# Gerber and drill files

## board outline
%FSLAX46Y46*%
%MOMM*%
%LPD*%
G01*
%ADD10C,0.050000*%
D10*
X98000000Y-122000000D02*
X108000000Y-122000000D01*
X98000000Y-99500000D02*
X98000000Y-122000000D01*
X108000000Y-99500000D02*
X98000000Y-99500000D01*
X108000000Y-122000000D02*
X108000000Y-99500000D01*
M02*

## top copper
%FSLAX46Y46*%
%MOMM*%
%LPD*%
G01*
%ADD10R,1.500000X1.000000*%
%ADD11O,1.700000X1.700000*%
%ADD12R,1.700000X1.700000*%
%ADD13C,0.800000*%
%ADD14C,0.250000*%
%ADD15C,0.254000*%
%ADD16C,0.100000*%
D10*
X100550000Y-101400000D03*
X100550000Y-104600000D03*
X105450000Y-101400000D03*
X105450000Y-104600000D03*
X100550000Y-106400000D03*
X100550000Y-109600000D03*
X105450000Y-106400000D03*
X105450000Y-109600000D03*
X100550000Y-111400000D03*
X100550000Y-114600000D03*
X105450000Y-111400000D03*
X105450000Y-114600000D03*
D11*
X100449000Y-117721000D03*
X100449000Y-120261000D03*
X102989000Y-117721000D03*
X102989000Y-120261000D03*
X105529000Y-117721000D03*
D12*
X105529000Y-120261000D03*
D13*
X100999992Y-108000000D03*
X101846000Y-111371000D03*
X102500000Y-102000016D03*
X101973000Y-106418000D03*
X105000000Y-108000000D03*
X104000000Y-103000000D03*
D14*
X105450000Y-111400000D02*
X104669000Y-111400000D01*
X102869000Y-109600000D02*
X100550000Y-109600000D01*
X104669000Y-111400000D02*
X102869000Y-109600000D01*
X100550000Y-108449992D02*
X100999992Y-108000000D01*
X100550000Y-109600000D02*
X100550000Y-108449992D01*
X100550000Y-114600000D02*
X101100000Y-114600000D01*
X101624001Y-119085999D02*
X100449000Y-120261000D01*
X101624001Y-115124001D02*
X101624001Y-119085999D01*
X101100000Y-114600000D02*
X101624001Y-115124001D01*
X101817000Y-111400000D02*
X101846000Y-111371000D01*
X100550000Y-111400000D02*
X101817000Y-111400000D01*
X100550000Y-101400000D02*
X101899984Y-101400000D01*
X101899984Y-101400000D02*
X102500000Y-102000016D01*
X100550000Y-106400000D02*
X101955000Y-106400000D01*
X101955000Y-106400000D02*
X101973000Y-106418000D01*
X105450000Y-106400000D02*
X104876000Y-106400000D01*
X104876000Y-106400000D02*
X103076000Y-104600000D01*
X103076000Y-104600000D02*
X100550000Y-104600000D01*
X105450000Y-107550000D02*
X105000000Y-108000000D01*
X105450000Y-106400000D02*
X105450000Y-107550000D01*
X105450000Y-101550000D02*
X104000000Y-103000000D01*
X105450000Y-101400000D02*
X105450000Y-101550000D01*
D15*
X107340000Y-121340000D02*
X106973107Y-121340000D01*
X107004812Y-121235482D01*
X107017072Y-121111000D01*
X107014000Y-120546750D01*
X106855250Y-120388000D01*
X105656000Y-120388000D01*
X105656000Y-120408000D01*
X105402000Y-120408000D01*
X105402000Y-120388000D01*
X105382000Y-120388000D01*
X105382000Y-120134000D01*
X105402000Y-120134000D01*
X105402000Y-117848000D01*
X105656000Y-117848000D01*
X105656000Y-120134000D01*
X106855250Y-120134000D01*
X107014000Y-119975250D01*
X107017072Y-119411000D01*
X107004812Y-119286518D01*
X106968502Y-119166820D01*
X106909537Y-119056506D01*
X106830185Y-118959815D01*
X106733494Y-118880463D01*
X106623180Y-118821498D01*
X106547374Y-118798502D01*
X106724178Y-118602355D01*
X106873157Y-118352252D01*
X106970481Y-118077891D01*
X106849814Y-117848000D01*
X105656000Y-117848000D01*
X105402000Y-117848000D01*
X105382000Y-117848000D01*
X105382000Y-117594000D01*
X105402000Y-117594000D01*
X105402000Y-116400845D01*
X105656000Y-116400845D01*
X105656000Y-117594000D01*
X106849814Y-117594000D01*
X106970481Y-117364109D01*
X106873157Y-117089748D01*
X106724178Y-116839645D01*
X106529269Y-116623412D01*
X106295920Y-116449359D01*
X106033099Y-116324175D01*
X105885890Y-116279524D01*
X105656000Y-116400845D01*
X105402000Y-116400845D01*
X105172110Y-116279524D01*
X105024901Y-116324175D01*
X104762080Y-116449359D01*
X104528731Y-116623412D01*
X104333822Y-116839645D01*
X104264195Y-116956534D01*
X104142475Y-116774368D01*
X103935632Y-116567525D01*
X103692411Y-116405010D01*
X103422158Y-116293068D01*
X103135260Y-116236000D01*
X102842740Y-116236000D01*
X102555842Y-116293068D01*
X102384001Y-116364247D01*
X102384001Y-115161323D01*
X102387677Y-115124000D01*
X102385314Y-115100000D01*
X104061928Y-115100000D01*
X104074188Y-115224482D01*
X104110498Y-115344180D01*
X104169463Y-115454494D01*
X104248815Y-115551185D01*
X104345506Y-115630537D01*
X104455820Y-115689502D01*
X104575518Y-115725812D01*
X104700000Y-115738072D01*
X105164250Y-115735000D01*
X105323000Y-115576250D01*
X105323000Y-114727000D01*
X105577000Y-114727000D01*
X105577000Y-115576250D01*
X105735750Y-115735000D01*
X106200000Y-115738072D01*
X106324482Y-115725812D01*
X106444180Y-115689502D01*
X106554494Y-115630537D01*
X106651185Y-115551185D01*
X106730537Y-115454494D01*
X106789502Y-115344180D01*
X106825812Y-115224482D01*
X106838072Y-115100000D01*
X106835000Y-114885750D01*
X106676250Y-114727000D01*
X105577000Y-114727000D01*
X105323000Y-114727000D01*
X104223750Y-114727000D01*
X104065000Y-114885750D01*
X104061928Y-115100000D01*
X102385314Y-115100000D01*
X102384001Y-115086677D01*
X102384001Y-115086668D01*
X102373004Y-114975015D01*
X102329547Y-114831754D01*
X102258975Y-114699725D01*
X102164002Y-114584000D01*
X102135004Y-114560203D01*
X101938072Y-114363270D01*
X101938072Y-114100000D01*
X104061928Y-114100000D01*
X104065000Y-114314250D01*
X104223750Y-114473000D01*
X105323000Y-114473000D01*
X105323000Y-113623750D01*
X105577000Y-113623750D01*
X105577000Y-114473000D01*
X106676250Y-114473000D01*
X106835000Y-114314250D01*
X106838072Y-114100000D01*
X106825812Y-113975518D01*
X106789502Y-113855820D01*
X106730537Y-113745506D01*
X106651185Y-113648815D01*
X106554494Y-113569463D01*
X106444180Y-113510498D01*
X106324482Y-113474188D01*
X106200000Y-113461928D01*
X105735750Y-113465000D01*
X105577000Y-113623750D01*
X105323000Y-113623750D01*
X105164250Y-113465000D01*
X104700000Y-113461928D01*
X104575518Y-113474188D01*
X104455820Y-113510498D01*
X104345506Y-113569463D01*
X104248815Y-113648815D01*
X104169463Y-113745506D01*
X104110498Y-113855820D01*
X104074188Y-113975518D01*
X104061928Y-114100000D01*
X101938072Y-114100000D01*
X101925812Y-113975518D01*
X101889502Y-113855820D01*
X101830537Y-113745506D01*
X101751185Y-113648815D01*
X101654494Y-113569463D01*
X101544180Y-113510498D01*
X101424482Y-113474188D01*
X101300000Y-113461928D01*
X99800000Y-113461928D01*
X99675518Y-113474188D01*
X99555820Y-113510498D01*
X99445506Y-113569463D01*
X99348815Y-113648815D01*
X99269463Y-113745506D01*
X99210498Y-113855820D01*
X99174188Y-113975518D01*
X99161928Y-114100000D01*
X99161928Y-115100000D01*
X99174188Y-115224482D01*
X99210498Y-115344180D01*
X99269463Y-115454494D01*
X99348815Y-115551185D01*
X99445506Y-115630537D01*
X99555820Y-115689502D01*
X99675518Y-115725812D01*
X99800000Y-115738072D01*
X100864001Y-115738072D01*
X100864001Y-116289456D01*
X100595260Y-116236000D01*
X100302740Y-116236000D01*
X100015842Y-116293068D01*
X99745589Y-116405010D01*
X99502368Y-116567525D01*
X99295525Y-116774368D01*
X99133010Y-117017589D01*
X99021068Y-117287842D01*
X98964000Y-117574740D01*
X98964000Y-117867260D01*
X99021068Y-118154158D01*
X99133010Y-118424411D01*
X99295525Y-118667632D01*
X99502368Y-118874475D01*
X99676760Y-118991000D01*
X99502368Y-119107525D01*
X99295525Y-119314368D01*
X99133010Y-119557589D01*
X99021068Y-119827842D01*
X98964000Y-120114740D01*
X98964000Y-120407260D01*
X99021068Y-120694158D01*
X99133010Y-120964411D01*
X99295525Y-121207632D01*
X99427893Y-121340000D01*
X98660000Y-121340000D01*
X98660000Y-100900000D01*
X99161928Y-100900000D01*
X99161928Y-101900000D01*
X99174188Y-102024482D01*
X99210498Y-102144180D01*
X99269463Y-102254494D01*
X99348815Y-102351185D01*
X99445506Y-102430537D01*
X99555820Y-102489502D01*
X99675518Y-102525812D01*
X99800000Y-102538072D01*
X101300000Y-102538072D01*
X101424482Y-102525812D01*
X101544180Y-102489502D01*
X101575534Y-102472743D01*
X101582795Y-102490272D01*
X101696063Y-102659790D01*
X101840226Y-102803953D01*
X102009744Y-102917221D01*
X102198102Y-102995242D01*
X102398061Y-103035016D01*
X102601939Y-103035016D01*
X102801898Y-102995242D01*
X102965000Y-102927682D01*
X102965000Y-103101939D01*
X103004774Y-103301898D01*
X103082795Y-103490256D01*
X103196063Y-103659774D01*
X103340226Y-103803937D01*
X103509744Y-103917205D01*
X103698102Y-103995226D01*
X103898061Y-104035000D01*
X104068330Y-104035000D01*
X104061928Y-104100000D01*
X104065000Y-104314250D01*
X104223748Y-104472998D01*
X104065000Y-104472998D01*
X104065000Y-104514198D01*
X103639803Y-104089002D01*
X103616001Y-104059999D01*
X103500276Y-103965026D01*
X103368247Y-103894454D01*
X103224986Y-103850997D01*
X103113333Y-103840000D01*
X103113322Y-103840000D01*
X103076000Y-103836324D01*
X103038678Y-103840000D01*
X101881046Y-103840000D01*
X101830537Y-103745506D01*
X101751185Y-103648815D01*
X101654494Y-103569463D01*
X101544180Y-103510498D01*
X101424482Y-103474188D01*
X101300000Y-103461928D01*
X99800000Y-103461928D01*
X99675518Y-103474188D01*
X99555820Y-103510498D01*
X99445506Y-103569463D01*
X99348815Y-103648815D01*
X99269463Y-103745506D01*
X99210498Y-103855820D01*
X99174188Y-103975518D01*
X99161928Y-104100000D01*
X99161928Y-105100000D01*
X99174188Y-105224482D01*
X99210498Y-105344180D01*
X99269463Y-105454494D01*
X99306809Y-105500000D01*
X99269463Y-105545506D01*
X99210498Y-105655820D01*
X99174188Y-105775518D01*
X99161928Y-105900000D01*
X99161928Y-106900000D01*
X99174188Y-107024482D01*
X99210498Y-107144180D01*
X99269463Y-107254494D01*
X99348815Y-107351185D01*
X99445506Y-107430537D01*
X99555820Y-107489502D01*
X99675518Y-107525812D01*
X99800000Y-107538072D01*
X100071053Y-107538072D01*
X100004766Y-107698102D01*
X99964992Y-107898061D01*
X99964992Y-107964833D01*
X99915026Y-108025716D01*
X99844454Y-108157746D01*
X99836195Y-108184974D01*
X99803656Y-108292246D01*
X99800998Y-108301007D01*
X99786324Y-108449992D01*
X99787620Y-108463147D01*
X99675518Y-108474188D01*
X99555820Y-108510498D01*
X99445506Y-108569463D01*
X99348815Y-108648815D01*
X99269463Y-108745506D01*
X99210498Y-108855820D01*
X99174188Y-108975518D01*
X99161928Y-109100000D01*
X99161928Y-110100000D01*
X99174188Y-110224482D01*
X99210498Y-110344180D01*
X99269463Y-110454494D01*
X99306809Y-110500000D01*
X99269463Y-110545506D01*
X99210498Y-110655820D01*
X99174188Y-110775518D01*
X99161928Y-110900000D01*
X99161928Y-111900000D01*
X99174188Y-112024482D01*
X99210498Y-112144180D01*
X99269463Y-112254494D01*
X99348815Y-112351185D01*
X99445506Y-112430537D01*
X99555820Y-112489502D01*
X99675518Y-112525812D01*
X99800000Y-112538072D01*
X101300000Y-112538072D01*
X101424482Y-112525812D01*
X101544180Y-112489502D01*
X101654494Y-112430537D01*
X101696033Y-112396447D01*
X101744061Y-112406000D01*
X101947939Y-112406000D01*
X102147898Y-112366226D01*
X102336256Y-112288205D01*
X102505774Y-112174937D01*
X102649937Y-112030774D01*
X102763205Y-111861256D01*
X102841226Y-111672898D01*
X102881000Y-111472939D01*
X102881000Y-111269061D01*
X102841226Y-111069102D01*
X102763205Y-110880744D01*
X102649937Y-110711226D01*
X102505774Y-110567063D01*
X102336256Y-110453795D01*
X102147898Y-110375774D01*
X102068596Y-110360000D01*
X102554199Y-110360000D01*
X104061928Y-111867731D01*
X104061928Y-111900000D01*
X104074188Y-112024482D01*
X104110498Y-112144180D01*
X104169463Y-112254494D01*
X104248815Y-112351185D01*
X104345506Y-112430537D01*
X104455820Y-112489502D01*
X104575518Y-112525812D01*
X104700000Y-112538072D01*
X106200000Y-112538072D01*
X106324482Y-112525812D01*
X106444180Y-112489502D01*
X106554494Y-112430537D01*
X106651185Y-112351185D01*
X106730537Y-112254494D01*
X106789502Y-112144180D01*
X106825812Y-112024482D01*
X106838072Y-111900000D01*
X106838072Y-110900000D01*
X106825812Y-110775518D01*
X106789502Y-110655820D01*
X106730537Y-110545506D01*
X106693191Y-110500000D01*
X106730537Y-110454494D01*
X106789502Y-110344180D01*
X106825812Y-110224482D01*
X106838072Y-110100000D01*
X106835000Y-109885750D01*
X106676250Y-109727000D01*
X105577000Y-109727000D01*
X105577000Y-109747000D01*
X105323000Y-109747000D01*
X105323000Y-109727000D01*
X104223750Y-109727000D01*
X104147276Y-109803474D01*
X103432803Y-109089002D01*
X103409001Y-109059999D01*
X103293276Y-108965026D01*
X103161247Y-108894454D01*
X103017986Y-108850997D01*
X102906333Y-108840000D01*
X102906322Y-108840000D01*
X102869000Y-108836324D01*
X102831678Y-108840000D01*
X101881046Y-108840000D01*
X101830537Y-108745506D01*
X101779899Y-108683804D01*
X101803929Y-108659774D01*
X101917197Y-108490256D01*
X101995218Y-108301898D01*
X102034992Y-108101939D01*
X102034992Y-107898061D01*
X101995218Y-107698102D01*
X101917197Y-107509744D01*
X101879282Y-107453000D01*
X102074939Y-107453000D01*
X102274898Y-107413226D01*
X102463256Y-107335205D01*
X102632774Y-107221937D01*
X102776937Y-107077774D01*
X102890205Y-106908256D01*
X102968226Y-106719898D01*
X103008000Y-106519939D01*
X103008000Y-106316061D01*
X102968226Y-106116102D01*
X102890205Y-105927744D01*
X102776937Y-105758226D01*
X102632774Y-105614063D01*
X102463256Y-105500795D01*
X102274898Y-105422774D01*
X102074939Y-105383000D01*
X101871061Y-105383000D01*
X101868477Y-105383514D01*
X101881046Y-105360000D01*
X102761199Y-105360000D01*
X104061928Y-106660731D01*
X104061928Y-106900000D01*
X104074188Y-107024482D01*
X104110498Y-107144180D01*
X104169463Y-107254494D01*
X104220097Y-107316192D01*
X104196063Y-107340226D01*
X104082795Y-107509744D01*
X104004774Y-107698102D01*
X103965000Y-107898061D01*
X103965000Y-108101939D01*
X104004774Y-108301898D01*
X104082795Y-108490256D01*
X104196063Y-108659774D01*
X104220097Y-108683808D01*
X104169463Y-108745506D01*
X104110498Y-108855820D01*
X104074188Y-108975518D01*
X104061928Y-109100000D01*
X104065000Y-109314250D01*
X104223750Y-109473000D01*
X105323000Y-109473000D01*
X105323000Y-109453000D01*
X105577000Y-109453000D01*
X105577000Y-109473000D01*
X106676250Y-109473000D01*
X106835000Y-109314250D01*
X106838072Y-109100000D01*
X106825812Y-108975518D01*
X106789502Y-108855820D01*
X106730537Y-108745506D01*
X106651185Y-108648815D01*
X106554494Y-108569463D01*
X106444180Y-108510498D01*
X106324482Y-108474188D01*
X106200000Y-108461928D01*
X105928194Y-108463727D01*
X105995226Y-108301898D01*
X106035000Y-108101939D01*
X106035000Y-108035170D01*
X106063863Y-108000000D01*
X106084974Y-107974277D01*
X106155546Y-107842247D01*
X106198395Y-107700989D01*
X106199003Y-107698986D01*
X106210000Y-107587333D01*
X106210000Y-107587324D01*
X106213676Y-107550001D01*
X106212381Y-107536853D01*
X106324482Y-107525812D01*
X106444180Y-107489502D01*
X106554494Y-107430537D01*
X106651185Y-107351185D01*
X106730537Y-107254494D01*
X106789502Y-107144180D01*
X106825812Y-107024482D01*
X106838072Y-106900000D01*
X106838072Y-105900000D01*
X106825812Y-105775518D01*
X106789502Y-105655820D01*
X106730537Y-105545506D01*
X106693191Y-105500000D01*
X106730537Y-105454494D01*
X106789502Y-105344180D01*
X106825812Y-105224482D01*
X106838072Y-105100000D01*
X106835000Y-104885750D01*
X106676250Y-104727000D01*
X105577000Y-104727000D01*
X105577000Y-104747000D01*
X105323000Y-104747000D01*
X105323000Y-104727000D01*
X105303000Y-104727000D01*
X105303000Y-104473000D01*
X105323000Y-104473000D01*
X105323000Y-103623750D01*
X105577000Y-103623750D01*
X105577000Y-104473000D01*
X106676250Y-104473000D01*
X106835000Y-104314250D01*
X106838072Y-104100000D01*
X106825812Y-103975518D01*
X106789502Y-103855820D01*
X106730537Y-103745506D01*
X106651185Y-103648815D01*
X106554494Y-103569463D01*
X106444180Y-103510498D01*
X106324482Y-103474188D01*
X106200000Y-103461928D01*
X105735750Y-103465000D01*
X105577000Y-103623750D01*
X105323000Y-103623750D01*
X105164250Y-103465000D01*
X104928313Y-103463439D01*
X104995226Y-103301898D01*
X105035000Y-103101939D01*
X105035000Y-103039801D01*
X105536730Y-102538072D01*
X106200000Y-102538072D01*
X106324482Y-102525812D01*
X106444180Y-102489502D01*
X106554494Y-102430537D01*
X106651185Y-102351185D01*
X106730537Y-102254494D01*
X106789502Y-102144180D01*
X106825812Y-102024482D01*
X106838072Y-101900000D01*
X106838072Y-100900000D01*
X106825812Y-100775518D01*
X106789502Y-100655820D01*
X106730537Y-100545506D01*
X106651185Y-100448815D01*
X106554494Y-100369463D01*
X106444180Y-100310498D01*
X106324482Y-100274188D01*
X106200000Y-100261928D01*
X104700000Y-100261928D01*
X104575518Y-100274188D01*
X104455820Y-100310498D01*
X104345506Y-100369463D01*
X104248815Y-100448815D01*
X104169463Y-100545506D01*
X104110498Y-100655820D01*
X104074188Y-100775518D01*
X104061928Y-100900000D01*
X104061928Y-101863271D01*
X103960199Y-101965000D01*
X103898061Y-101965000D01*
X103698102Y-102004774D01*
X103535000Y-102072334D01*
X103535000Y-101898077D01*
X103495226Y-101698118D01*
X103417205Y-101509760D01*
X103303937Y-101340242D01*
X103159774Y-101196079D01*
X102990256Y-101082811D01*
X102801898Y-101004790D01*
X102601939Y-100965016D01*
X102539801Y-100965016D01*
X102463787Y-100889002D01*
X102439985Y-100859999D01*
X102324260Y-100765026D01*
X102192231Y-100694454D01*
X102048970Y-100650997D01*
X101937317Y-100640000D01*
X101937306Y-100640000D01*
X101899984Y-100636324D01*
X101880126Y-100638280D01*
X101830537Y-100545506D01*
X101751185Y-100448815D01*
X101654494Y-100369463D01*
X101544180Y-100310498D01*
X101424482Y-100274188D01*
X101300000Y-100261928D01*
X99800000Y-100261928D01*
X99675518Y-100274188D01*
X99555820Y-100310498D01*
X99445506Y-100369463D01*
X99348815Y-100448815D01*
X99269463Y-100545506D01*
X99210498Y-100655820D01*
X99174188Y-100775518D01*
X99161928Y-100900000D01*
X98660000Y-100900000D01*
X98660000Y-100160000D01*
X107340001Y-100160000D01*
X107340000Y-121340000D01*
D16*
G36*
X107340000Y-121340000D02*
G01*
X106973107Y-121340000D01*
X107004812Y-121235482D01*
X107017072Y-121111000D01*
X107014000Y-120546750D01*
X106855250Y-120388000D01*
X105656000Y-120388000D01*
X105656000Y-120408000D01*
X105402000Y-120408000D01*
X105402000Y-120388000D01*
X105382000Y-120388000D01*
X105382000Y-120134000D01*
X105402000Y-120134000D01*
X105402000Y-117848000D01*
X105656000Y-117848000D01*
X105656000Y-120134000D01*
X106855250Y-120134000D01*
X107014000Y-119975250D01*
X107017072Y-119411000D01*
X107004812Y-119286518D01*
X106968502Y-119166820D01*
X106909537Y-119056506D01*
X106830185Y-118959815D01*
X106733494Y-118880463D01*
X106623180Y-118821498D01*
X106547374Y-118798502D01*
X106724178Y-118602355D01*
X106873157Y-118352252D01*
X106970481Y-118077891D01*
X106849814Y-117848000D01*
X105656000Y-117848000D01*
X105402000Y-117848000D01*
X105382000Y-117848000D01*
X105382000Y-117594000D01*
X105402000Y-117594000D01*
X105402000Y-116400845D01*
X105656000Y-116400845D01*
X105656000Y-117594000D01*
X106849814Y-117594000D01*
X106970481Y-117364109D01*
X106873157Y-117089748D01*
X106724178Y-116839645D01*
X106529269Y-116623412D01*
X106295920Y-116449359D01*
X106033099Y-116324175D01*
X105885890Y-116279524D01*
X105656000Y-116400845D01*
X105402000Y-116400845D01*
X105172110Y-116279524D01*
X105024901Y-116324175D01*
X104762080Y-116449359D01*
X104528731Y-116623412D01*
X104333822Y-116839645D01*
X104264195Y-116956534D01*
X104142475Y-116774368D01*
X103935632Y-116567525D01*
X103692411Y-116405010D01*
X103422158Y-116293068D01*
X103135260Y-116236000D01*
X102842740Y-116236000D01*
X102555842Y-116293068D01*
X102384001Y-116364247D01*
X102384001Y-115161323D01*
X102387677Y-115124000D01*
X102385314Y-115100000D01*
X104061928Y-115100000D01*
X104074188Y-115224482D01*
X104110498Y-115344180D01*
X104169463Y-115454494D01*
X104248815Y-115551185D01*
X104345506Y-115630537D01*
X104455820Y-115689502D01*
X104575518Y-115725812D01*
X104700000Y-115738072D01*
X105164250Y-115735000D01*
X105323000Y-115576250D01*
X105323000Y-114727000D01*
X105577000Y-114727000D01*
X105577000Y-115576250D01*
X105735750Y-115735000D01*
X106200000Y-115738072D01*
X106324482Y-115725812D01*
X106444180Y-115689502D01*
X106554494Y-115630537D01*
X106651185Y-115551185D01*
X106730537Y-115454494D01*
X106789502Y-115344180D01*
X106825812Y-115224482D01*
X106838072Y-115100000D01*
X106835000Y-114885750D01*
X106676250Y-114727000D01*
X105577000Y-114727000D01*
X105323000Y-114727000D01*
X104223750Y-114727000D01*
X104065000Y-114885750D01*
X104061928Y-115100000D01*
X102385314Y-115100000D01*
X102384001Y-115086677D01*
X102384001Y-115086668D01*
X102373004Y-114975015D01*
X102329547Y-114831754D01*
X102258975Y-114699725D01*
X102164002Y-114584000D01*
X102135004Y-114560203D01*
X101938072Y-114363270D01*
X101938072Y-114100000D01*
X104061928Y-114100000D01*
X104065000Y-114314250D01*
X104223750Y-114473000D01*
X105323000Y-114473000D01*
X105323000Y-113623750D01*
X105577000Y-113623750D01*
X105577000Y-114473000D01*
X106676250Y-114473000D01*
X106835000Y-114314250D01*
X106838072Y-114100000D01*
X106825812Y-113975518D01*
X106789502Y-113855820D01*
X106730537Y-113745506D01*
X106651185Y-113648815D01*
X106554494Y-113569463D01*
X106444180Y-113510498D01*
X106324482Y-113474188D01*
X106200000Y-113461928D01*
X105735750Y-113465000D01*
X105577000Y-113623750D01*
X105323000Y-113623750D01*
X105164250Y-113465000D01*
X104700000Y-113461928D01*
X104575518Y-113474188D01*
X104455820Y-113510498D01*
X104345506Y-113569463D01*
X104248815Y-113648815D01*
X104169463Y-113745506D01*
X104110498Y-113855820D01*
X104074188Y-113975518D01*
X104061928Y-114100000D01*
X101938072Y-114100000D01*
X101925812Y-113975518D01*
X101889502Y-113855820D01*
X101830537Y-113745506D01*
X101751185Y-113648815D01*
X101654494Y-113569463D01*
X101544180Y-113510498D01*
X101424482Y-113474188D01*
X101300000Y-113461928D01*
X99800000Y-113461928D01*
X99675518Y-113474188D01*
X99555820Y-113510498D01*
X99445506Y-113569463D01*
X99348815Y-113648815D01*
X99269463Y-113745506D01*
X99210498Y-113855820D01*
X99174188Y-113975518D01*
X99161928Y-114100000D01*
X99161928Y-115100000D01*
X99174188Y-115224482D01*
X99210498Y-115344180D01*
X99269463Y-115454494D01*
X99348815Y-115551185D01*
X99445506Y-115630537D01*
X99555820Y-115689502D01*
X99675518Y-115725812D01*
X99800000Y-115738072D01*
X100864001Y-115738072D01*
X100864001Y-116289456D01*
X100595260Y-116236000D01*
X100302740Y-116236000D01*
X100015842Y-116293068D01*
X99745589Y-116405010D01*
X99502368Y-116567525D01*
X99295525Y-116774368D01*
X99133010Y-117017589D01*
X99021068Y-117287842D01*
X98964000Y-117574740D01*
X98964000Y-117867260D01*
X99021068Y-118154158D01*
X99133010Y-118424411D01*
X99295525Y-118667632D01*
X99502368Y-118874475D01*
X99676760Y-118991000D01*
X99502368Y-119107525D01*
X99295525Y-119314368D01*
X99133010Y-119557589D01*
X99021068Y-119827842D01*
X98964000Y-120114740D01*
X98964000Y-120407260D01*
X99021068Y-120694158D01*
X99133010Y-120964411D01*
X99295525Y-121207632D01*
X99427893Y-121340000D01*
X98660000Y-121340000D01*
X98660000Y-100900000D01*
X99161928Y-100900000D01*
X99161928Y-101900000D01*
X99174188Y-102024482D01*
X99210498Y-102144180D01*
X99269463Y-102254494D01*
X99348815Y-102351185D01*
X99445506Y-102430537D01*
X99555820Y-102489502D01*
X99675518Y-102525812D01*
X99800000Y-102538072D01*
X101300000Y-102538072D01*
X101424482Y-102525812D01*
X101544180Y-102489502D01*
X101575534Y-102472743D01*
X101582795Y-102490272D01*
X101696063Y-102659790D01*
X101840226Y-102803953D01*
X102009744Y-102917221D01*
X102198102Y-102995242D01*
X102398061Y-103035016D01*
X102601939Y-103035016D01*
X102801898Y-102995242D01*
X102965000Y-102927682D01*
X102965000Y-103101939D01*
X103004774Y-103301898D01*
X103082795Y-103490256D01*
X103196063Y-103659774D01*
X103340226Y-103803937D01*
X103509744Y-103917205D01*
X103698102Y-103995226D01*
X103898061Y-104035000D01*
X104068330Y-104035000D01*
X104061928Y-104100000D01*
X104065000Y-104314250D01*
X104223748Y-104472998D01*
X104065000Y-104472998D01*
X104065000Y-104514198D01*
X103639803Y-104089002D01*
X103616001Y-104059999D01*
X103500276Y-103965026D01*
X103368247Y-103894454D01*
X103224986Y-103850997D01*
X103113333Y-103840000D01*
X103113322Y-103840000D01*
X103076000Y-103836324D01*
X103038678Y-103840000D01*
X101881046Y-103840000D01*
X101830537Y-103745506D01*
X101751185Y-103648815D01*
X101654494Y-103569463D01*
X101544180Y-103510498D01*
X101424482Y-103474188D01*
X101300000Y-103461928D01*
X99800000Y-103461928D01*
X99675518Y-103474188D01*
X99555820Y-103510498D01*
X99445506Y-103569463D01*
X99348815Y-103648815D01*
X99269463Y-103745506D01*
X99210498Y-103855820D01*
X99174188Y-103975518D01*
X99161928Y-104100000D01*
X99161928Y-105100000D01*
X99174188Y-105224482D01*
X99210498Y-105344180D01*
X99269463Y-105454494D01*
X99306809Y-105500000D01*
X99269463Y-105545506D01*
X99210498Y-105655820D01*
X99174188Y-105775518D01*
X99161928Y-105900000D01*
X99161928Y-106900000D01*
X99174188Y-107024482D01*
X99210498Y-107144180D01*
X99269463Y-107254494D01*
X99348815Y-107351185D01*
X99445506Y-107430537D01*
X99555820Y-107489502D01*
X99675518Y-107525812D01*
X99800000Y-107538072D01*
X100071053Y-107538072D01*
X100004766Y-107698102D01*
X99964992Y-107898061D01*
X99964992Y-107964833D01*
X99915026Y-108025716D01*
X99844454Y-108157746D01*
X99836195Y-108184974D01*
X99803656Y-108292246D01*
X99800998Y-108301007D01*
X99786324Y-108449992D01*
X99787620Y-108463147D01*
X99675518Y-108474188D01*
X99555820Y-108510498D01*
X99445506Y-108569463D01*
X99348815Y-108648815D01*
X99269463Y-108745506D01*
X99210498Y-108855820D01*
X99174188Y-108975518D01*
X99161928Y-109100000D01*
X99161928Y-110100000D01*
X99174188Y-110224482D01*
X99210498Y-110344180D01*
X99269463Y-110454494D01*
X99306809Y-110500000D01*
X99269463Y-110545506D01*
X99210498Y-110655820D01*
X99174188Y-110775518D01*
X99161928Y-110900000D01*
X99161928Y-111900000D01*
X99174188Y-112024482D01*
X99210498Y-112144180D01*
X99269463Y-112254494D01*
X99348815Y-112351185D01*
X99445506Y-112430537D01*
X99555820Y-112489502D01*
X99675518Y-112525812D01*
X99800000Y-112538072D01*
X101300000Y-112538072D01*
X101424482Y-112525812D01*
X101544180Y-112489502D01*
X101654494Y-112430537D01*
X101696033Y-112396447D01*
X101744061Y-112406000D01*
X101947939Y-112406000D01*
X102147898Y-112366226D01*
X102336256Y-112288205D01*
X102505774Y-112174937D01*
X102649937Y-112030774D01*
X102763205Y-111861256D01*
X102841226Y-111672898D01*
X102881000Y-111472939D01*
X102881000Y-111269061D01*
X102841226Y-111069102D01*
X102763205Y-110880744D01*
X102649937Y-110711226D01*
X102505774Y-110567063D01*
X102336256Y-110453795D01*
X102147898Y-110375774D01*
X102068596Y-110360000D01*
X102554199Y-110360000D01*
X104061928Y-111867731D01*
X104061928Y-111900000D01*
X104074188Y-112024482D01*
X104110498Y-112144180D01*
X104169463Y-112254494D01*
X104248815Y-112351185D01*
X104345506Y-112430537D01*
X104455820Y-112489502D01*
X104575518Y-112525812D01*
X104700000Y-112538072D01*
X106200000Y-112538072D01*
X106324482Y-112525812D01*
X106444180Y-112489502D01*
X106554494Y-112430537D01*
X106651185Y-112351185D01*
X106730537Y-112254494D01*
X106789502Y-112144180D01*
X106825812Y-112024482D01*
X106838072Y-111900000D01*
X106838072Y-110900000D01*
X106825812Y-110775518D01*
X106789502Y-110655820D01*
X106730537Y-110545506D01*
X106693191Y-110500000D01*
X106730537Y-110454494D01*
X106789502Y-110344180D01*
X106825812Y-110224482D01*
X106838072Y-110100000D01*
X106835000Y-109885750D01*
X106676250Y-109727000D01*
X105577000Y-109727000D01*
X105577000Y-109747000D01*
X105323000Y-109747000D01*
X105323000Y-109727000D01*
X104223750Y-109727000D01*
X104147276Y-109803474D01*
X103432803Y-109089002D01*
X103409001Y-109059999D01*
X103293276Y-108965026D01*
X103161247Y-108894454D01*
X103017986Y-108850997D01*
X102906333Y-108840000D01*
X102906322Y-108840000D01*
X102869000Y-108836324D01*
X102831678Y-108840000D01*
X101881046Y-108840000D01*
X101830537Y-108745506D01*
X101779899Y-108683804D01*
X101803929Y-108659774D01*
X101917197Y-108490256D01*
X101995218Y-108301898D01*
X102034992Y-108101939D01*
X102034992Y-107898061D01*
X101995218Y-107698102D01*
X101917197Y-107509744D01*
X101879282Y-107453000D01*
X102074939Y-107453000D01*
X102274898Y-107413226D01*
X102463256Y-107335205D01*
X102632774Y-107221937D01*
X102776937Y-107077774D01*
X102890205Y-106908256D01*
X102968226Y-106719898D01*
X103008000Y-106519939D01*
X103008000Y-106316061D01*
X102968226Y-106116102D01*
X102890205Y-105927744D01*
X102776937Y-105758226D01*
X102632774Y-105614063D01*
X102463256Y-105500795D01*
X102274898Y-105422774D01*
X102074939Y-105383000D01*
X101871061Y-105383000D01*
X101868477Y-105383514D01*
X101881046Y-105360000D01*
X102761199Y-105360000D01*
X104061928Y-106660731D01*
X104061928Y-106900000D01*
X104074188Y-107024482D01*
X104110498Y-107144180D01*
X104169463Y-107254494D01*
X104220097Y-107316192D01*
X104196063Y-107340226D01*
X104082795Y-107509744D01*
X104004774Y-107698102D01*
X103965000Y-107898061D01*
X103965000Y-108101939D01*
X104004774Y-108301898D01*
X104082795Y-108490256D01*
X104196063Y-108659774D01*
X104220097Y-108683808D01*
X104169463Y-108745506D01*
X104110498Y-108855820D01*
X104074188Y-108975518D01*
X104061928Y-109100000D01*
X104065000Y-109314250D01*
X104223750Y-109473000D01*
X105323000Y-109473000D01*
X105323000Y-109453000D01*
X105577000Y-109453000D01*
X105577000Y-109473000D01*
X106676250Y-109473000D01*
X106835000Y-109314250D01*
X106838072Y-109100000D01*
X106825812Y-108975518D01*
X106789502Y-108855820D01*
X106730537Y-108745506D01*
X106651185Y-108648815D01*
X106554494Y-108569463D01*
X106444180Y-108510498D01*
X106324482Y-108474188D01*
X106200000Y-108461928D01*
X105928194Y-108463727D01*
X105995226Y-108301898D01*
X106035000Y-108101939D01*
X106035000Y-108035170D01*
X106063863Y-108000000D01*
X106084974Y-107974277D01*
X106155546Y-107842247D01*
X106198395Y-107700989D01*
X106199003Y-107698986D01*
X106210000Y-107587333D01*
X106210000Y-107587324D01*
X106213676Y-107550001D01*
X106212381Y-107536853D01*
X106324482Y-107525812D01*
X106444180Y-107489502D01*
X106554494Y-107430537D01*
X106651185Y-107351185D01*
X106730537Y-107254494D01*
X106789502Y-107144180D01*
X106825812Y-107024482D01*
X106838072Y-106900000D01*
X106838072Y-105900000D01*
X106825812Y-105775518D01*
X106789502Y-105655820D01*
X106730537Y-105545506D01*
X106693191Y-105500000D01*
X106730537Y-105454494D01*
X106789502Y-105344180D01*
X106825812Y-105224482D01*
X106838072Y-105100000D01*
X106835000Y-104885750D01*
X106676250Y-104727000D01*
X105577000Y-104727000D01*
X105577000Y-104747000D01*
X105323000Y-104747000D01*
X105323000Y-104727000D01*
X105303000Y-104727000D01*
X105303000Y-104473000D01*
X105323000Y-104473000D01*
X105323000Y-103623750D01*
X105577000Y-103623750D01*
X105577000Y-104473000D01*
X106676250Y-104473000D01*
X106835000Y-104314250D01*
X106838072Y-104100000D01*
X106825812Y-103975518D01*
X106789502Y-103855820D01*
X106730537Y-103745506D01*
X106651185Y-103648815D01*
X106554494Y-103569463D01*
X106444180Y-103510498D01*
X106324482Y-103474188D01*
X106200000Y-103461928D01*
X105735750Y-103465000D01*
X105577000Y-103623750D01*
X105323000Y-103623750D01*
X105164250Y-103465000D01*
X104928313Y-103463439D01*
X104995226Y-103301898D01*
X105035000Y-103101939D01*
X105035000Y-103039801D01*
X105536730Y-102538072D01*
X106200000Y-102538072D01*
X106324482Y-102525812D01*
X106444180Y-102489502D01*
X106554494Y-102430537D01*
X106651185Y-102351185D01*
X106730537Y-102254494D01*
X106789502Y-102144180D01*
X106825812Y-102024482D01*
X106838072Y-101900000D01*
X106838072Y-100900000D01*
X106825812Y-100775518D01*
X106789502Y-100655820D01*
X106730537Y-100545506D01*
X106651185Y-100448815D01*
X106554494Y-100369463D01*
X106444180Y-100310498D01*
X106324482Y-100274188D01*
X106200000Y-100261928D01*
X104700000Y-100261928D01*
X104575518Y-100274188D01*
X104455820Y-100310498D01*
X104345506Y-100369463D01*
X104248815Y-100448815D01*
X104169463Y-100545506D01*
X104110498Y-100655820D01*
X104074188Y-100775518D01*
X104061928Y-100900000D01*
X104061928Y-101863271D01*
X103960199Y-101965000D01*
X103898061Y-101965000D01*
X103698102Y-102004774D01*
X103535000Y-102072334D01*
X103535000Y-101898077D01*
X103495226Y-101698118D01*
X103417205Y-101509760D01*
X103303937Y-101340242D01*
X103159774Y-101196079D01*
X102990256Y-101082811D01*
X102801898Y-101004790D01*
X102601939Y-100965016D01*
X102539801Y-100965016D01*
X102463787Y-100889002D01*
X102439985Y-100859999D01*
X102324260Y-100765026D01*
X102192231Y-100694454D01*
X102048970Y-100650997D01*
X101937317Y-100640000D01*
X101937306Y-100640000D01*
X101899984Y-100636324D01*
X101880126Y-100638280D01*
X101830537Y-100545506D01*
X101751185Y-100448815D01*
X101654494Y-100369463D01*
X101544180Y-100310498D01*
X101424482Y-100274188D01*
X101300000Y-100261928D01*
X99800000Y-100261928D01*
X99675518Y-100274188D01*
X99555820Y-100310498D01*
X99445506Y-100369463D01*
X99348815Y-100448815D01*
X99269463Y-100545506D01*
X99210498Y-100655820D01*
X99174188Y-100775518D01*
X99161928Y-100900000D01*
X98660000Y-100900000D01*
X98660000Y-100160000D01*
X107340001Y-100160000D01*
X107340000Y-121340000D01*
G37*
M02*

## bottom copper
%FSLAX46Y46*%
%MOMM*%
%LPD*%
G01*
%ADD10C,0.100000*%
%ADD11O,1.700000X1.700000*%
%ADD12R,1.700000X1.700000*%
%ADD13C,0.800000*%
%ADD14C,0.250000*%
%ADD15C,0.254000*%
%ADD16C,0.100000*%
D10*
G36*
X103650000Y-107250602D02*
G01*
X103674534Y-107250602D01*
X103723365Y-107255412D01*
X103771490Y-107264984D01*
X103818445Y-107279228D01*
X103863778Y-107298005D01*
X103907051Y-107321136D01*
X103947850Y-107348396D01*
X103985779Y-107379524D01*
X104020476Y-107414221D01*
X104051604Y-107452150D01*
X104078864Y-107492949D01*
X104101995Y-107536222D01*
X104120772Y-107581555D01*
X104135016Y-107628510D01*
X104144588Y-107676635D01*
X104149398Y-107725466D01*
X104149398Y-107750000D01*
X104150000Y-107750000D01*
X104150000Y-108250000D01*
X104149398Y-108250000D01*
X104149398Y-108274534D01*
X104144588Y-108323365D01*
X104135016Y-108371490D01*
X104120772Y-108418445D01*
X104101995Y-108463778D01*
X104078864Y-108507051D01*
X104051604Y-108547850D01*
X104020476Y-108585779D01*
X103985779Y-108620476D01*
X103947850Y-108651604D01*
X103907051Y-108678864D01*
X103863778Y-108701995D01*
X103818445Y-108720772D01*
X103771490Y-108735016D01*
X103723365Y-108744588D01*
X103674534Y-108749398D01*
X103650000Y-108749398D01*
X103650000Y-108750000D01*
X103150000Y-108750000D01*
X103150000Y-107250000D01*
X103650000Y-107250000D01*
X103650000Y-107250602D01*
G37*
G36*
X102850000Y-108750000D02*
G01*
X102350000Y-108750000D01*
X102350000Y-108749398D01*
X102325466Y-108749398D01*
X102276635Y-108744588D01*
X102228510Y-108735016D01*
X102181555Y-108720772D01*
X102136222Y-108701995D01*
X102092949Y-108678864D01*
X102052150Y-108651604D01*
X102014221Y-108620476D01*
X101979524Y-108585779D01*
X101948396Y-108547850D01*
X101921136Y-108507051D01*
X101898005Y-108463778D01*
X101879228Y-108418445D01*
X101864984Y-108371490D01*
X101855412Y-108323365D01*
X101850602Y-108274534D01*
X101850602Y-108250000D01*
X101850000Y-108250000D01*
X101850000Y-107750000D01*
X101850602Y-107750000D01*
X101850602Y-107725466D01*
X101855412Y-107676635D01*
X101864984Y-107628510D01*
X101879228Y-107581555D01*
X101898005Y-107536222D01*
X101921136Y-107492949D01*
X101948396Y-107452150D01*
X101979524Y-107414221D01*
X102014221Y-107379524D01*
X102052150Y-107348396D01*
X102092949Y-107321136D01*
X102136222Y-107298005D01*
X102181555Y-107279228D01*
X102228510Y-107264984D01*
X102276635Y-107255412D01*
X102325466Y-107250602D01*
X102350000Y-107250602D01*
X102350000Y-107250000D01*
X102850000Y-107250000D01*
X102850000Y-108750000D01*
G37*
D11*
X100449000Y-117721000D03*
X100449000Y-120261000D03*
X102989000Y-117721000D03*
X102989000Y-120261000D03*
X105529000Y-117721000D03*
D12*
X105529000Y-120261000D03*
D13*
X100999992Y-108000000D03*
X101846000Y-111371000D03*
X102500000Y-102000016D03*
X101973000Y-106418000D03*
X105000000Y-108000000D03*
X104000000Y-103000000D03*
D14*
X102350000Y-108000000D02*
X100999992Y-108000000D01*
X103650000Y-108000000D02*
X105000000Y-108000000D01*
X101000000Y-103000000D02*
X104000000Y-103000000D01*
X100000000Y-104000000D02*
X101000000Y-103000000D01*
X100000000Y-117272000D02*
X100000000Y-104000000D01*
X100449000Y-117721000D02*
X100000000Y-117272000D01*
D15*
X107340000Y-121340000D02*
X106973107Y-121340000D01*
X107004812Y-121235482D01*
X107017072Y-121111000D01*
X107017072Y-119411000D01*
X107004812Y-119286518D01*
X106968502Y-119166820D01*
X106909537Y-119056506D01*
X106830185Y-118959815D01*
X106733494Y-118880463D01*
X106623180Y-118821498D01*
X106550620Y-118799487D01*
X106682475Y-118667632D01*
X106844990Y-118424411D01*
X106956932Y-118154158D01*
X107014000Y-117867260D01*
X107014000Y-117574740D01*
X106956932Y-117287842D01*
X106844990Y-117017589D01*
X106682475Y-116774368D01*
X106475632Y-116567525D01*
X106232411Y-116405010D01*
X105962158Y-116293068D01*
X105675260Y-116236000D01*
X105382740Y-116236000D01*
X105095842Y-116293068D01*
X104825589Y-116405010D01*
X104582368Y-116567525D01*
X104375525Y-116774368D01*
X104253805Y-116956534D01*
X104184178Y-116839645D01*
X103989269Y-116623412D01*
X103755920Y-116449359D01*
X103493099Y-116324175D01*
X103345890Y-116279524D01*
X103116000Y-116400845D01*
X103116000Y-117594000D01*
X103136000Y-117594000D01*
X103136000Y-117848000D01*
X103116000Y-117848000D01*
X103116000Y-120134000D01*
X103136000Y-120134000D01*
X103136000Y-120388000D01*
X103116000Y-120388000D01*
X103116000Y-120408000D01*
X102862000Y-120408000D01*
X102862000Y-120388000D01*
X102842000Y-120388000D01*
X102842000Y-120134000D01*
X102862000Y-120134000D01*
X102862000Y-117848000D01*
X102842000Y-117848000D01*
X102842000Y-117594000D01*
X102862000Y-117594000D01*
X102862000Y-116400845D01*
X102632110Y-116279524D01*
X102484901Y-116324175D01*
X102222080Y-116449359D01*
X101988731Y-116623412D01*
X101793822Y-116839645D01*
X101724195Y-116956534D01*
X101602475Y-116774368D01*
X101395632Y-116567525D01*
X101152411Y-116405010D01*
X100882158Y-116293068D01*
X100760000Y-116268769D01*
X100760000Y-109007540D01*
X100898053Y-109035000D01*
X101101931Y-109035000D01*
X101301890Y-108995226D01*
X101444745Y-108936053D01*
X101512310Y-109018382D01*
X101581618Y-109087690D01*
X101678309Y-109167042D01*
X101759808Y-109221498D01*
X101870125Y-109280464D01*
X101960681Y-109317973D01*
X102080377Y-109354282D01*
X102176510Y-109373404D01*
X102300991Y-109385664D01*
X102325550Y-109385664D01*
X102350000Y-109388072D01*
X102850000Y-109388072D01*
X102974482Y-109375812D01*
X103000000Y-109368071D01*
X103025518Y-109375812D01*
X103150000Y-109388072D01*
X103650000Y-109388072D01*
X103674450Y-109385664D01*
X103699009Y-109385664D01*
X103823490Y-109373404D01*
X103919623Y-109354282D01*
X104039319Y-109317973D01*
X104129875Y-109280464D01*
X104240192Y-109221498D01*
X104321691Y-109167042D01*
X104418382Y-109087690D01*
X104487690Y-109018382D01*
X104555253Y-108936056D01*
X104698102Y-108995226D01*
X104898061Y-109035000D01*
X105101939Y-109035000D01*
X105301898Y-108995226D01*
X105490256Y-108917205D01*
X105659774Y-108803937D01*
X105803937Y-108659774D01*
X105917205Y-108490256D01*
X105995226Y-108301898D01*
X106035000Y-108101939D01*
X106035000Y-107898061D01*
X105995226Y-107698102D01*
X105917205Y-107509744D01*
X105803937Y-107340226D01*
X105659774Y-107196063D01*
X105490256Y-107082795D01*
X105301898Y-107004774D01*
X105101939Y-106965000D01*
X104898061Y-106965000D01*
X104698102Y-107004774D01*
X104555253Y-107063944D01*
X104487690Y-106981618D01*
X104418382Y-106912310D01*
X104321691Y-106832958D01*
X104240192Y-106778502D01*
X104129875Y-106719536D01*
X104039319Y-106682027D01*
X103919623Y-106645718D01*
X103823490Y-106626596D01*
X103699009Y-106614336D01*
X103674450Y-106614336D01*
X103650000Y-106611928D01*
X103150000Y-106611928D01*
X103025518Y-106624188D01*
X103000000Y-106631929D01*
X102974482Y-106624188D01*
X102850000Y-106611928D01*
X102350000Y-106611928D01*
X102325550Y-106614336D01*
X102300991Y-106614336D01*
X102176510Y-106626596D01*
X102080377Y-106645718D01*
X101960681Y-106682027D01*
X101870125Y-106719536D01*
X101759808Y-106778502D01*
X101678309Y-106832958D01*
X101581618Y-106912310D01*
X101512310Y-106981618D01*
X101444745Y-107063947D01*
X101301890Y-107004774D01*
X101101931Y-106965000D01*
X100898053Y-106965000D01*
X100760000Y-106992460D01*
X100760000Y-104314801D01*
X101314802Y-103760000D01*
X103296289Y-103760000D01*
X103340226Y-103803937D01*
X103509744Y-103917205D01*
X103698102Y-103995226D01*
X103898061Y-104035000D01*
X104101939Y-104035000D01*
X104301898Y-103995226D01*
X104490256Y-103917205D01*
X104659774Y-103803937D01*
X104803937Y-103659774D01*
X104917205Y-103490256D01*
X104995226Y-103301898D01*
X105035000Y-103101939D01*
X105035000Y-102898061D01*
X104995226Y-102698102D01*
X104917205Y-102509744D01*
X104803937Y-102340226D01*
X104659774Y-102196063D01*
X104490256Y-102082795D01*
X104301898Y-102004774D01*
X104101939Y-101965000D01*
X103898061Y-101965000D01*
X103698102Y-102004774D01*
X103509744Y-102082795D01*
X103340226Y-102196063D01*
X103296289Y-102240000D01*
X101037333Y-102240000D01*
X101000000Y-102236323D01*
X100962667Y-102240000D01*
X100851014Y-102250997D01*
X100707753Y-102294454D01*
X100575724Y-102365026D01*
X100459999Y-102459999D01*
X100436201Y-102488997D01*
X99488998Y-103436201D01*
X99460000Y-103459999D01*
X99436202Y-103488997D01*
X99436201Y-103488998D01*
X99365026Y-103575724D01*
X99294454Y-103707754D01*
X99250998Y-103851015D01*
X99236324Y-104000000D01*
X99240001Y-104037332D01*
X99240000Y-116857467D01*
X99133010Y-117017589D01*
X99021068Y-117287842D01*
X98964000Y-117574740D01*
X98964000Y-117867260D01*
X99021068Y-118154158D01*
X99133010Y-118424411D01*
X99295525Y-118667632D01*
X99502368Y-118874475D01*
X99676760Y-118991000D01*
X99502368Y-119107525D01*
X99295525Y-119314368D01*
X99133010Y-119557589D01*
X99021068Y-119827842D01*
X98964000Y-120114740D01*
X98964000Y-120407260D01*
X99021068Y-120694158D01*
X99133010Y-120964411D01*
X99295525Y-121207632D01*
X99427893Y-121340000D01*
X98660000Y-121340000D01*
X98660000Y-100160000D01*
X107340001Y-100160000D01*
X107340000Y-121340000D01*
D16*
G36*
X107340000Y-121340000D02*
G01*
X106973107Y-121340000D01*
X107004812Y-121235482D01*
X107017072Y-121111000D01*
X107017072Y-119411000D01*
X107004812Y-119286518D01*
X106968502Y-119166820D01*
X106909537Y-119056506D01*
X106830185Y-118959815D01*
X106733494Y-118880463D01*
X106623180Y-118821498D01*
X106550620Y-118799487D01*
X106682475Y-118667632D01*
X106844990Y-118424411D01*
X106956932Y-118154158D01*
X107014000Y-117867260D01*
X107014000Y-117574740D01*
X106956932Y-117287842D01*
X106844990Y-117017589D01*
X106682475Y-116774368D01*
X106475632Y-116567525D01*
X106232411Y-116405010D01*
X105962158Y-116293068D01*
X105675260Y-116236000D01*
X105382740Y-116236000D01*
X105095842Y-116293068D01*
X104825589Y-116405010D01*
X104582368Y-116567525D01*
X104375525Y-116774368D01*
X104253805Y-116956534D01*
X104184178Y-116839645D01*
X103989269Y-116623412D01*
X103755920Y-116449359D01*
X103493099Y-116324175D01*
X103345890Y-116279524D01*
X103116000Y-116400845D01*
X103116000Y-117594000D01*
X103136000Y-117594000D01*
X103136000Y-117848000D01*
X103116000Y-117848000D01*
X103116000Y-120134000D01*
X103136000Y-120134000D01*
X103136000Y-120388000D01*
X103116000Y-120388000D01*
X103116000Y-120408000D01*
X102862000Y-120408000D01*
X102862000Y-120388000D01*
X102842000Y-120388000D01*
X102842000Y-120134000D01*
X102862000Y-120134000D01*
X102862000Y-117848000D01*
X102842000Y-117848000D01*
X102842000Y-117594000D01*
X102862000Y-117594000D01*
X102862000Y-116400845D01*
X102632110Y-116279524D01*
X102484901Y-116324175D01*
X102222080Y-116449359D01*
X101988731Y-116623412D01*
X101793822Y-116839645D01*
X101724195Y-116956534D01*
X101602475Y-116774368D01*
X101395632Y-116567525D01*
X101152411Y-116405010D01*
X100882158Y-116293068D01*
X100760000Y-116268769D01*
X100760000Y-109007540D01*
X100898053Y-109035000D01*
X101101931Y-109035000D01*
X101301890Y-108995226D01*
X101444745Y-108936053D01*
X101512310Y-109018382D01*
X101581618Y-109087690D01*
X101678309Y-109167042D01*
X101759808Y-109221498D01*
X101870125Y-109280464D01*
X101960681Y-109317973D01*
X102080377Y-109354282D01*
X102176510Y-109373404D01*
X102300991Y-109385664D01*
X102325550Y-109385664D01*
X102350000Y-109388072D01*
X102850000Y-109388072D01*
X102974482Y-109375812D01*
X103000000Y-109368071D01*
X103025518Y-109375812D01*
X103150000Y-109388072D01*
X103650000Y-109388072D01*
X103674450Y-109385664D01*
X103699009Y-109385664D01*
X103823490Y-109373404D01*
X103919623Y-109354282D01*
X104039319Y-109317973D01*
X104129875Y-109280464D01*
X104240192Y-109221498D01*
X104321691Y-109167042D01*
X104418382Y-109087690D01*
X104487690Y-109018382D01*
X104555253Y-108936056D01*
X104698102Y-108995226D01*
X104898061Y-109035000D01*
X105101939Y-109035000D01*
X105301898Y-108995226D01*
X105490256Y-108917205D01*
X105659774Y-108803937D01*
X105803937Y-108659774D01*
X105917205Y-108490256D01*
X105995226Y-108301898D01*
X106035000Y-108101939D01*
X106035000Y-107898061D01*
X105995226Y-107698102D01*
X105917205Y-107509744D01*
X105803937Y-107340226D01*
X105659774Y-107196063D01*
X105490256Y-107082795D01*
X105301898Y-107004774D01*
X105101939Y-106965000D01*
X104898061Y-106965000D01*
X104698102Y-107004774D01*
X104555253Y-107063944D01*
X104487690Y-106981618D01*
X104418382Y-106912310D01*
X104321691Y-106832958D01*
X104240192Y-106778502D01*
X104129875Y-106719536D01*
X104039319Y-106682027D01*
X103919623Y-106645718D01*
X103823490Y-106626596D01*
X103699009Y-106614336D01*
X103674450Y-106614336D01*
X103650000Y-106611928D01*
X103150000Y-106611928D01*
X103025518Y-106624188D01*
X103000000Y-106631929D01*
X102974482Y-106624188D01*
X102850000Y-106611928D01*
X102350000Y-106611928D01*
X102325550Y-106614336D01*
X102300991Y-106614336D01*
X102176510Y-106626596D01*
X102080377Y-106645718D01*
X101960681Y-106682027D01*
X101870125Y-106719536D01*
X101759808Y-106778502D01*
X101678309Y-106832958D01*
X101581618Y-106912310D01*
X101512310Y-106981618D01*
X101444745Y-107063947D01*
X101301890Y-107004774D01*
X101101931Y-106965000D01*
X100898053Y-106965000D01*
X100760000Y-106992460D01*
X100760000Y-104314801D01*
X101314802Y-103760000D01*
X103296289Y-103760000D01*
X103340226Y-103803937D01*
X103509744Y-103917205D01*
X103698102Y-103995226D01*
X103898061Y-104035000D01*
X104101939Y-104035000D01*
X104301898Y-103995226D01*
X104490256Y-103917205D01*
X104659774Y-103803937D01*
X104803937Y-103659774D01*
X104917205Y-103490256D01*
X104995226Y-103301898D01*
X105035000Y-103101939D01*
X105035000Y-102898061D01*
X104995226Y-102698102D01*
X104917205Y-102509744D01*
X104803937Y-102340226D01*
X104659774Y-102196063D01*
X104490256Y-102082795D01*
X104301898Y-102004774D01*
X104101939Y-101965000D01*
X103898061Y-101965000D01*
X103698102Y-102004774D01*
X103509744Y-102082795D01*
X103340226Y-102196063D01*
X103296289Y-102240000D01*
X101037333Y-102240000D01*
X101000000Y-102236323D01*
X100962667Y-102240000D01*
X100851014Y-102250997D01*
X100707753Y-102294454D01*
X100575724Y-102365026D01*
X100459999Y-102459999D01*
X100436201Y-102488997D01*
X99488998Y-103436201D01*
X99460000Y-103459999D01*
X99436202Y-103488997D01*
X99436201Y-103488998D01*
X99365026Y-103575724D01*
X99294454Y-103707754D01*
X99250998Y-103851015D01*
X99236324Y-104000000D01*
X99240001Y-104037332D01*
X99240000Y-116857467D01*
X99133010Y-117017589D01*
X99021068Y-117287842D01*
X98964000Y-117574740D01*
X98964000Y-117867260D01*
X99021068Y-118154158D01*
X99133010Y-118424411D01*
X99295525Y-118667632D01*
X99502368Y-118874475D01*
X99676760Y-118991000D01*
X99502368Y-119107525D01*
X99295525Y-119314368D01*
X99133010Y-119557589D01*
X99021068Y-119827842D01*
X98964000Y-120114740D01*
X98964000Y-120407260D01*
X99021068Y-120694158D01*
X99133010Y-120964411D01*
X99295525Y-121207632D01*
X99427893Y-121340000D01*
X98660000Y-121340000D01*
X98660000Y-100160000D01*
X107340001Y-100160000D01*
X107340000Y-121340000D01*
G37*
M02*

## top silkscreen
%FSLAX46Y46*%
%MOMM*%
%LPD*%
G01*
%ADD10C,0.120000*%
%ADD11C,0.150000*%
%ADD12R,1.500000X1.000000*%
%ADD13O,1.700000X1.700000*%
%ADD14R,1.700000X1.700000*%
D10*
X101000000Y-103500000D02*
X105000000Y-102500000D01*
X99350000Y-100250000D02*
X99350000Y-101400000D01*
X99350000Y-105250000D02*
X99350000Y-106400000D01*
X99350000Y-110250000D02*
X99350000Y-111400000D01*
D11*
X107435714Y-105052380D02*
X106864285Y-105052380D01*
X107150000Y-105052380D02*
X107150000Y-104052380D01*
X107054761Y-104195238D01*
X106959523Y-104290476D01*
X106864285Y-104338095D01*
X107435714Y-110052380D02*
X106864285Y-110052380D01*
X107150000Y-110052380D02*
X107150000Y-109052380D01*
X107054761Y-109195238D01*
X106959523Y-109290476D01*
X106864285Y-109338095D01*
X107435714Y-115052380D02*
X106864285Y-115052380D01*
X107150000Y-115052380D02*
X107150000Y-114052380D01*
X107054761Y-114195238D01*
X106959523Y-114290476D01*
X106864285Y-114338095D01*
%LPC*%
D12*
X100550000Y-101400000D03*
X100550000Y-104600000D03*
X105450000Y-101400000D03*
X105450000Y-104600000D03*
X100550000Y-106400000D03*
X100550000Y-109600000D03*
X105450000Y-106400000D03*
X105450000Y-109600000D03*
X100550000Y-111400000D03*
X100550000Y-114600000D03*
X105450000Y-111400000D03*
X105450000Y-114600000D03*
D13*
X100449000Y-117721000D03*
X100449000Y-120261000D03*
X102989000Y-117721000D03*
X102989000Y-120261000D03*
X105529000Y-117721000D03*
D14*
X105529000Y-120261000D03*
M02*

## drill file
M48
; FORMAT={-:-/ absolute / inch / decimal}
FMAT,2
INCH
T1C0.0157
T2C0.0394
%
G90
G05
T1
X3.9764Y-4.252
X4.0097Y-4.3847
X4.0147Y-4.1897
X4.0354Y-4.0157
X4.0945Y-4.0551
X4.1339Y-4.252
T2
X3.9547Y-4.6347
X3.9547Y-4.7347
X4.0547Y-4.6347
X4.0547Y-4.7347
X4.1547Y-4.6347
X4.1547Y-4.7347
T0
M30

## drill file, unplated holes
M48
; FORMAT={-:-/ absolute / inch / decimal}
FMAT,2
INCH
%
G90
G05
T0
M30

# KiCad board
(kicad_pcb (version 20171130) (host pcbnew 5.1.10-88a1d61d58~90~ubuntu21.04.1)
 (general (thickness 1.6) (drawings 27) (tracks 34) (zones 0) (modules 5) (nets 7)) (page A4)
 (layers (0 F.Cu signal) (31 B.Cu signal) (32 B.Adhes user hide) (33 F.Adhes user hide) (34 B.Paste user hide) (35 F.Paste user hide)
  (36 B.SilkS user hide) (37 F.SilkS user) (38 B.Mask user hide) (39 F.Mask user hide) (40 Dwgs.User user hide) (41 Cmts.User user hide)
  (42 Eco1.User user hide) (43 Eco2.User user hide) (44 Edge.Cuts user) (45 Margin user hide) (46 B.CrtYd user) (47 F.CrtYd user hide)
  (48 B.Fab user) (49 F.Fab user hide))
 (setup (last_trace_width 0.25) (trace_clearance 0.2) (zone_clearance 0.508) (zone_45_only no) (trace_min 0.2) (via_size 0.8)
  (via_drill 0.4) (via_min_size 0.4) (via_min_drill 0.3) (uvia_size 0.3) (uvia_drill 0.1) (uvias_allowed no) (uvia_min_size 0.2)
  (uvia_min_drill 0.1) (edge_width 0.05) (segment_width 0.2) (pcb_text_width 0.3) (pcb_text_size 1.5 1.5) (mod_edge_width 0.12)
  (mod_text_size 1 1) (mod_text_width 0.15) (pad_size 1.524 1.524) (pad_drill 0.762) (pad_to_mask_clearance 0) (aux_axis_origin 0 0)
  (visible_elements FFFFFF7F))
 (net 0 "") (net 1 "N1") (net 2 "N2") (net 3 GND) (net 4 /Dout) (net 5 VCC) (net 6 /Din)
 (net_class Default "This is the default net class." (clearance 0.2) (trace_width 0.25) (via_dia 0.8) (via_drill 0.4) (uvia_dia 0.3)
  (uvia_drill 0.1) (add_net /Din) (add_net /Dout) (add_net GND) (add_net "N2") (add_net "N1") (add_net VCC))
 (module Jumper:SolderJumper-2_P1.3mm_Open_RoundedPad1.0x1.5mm (layer B.Cu) (at 103 108)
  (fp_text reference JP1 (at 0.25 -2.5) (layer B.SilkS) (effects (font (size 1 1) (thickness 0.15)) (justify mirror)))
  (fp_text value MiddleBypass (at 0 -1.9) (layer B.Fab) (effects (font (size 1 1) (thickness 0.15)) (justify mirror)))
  (pad 2 smd custom (at 0.65 0) (size 1 0.5) (layers B.Cu B.Mask) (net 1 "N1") (zone_connect 2) (options (clearance outline) (anchor rect))
   (primitives))
  (pad 1 smd custom (at -0.65 0) (size 1 0.5) (layers B.Cu B.Mask) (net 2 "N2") (zone_connect 2) (options (clearance outline) (anchor rect))
   (primitives)))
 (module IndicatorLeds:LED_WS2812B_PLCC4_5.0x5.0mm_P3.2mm (layer F.Cu) (at 103 103 180)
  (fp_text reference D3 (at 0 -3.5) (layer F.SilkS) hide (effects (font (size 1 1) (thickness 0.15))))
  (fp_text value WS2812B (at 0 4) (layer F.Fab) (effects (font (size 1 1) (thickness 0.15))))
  (fp_line (start 3.65 2.75) (end 3.65 1.6) (layer F.SilkS) (width 0.12))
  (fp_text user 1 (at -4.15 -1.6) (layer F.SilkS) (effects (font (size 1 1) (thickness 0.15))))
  (pad 3 smd rect (at 2.45 1.6 180) (size 1.5 1) (layers F.Cu F.Paste F.Mask) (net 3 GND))
  (pad 4 smd rect (at 2.45 -1.6 180) (size 1.5 1) (layers F.Cu F.Paste F.Mask) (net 1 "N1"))
  (pad 2 smd rect (at -2.45 1.6 180) (size 1.5 1) (layers F.Cu F.Paste F.Mask) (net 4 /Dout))
  (pad 1 smd rect (at -2.45 -1.6 180) (size 1.5 1) (layers F.Cu F.Paste F.Mask) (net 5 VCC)))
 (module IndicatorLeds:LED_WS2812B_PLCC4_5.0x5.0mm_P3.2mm (layer F.Cu) (at 103 108 180)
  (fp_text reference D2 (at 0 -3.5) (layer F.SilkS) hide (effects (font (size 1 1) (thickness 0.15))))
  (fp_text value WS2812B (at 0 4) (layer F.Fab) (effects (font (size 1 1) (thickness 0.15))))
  (fp_line (start 3.65 2.75) (end 3.65 1.6) (layer F.SilkS) (width 0.12))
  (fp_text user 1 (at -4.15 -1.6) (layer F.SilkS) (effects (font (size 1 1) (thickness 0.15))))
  (pad 3 smd rect (at 2.45 1.6 180) (size 1.5 1) (layers F.Cu F.Paste F.Mask) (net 3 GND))
  (pad 4 smd rect (at 2.45 -1.6 180) (size 1.5 1) (layers F.Cu F.Paste F.Mask) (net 2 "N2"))
  (pad 2 smd rect (at -2.45 1.6 180) (size 1.5 1) (layers F.Cu F.Paste F.Mask) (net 1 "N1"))
  (pad 1 smd rect (at -2.45 -1.6 180) (size 1.5 1) (layers F.Cu F.Paste F.Mask) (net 5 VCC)))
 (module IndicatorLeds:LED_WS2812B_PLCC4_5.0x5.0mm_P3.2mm (layer F.Cu) (at 103 113 180)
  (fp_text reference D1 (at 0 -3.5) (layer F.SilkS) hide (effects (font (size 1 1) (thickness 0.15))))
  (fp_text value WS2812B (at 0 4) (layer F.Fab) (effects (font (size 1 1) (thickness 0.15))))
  (fp_line (start 3.65 2.75) (end 3.65 1.6) (layer F.SilkS) (width 0.12))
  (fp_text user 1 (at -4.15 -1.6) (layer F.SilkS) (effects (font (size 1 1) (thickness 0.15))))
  (pad 3 smd rect (at 2.45 1.6 180) (size 1.5 1) (layers F.Cu F.Paste F.Mask) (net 3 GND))
  (pad 4 smd rect (at 2.45 -1.6 180) (size 1.5 1) (layers F.Cu F.Paste F.Mask) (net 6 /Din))
  (pad 2 smd rect (at -2.45 1.6 180) (size 1.5 1) (layers F.Cu F.Paste F.Mask) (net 2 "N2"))
  (pad 1 smd rect (at -2.45 -1.6 180) (size 1.5 1) (layers F.Cu F.Paste F.Mask) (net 5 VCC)))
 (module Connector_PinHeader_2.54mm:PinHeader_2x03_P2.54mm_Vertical (layer B.Cu) (at 105.529 120.261 90)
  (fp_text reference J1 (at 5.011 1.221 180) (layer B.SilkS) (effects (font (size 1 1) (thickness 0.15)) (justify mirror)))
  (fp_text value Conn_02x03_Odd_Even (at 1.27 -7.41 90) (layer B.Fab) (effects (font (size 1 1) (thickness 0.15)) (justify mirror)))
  (pad 6 thru_hole oval (at 2.54 -5.08 90) (size 1.7 1.7) (drill 1) (layers *.Cu *.Mask) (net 4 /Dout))
  (pad 5 thru_hole oval (at 0 -5.08 90) (size 1.7 1.7) (drill 1) (layers *.Cu *.Mask) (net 6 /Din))
  (pad 4 thru_hole oval (at 2.54 -2.54 90) (size 1.7 1.7) (drill 1) (layers *.Cu *.Mask) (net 3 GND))
  (pad 3 thru_hole oval (at 0 -2.54 90) (size 1.7 1.7) (drill 1) (layers *.Cu *.Mask) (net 3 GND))
  (pad 2 thru_hole oval (at 2.54 0 90) (size 1.7 1.7) (drill 1) (layers *.Cu *.Mask) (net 5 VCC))
  (pad 1 thru_hole rect (at 0 0 90) (size 1.7 1.7) (drill 1) (layers *.Cu *.Mask) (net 5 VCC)))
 (gr_line (start 101 103.5) (end 105 102.5) (layer F.SilkS) (width 0.12))
 (gr_line (start 98 122) (end 108 122) (layer Edge.Cuts) (width 0.05))
 (gr_line (start 98 99.5) (end 98 122) (layer Edge.Cuts) (width 0.05))
 (gr_line (start 108 99.5) (end 98 99.5) (layer Edge.Cuts) (width 0.05))
 (gr_line (start 108 122) (end 108 99.5) (layer Edge.Cuts) (width 0.05))
 (segment (start 105.45 111.4) (end 104.669 111.4) (width 0.25) (layer F.Cu) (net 2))
 (segment (start 102.869 109.6) (end 100.55 109.6) (width 0.25) (layer F.Cu) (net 2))
 (segment (start 104.669 111.4) (end 102.869 109.6) (width 0.25) (layer F.Cu) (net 2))
 (via (at 100.999992 108) (size 0.8) (drill 0.4) (layers F.Cu B.Cu) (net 2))
 (segment (start 102.35 108) (end 100.999992 108) (width 0.25) (layer B.Cu) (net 2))
 (segment (start 100.55 108.449992) (end 100.999992 108) (width 0.25) (layer F.Cu) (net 2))
 (segment (start 100.55 109.6) (end 100.55 108.449992) (width 0.25) (layer F.Cu) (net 2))
 (segment (start 100.55 114.6) (end 101.1 114.6) (width 0.25) (layer F.Cu) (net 6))
 (segment (start 101.624001 119.085999) (end 100.449 120.261) (width 0.25) (layer F.Cu) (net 6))
 (segment (start 101.624001 115.124001) (end 101.624001 119.085999) (width 0.25) (layer F.Cu) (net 6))
 (segment (start 101.1 114.6) (end 101.624001 115.124001) (width 0.25) (layer F.Cu) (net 6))
 (via (at 101.846 111.371) (size 0.8) (drill 0.4) (layers F.Cu B.Cu) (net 3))
 (segment (start 101.817 111.4) (end 101.846 111.371) (width 0.25) (layer F.Cu) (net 3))
 (segment (start 100.55 111.4) (end 101.817 111.4) (width 0.25) (layer F.Cu) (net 3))
 (via (at 102.5 102.000016) (size 0.8) (drill 0.4) (layers F.Cu B.Cu) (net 3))
 (segment (start 100.55 101.4) (end 101.899984 101.4) (width 0.25) (layer F.Cu) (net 3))
 (segment (start 101.899984 101.4) (end 102.5 102.000016) (width 0.25) (layer F.Cu) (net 3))
 (via (at 101.973 106.418) (size 0.8) (drill 0.4) (layers F.Cu B.Cu) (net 3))
 (segment (start 100.55 106.4) (end 101.955 106.4) (width 0.25) (layer F.Cu) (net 3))
 (segment (start 101.955 106.4) (end 101.973 106.418) (width 0.25) (layer F.Cu) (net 3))
 (segment (start 105.45 106.4) (end 104.876 106.4) (width 0.25) (layer F.Cu) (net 1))
 (segment (start 104.876 106.4) (end 103.076 104.6) (width 0.25) (layer F.Cu) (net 1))
 (segment (start 103.076 104.6) (end 100.55 104.6) (width 0.25) (layer F.Cu) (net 1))
 (segment (start 105.45 107.55) (end 105 108) (width 0.25) (layer F.Cu) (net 1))
 (segment (start 105.45 106.4) (end 105.45 107.55) (width 0.25) (layer F.Cu) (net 1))
 (segment (start 103.65 108) (end 105 108) (width 0.25) (layer B.Cu) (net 1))
 (via (at 105 108) (size 0.8) (drill 0.4) (layers F.Cu B.Cu) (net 1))
 (via (at 104 103) (size 0.8) (drill 0.4) (layers F.Cu B.Cu) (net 4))
 (segment (start 105.45 101.55) (end 104 103) (width 0.25) (layer F.Cu) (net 4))
 (segment (start 105.45 101.4) (end 105.45 101.55) (width 0.25) (layer F.Cu) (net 4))
 (segment (start 101 103) (end 104 103) (width 0.25) (layer B.Cu) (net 4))
 (segment (start 100 104) (end 101 103) (width 0.25) (layer B.Cu) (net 4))
 (segment (start 100 117.272) (end 100 104) (width 0.25) (layer B.Cu) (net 4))
 (segment (start 100.449 117.721) (end 100 117.272) (width 0.25) (layer B.Cu) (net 4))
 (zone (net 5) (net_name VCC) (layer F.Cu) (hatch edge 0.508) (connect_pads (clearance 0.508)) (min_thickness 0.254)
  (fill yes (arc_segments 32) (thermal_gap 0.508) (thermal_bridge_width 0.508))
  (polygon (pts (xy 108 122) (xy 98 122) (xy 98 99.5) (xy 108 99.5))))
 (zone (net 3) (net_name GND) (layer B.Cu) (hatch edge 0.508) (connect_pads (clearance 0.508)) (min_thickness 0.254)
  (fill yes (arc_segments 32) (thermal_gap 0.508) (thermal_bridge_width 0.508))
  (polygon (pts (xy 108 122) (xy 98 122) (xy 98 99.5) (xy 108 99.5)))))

